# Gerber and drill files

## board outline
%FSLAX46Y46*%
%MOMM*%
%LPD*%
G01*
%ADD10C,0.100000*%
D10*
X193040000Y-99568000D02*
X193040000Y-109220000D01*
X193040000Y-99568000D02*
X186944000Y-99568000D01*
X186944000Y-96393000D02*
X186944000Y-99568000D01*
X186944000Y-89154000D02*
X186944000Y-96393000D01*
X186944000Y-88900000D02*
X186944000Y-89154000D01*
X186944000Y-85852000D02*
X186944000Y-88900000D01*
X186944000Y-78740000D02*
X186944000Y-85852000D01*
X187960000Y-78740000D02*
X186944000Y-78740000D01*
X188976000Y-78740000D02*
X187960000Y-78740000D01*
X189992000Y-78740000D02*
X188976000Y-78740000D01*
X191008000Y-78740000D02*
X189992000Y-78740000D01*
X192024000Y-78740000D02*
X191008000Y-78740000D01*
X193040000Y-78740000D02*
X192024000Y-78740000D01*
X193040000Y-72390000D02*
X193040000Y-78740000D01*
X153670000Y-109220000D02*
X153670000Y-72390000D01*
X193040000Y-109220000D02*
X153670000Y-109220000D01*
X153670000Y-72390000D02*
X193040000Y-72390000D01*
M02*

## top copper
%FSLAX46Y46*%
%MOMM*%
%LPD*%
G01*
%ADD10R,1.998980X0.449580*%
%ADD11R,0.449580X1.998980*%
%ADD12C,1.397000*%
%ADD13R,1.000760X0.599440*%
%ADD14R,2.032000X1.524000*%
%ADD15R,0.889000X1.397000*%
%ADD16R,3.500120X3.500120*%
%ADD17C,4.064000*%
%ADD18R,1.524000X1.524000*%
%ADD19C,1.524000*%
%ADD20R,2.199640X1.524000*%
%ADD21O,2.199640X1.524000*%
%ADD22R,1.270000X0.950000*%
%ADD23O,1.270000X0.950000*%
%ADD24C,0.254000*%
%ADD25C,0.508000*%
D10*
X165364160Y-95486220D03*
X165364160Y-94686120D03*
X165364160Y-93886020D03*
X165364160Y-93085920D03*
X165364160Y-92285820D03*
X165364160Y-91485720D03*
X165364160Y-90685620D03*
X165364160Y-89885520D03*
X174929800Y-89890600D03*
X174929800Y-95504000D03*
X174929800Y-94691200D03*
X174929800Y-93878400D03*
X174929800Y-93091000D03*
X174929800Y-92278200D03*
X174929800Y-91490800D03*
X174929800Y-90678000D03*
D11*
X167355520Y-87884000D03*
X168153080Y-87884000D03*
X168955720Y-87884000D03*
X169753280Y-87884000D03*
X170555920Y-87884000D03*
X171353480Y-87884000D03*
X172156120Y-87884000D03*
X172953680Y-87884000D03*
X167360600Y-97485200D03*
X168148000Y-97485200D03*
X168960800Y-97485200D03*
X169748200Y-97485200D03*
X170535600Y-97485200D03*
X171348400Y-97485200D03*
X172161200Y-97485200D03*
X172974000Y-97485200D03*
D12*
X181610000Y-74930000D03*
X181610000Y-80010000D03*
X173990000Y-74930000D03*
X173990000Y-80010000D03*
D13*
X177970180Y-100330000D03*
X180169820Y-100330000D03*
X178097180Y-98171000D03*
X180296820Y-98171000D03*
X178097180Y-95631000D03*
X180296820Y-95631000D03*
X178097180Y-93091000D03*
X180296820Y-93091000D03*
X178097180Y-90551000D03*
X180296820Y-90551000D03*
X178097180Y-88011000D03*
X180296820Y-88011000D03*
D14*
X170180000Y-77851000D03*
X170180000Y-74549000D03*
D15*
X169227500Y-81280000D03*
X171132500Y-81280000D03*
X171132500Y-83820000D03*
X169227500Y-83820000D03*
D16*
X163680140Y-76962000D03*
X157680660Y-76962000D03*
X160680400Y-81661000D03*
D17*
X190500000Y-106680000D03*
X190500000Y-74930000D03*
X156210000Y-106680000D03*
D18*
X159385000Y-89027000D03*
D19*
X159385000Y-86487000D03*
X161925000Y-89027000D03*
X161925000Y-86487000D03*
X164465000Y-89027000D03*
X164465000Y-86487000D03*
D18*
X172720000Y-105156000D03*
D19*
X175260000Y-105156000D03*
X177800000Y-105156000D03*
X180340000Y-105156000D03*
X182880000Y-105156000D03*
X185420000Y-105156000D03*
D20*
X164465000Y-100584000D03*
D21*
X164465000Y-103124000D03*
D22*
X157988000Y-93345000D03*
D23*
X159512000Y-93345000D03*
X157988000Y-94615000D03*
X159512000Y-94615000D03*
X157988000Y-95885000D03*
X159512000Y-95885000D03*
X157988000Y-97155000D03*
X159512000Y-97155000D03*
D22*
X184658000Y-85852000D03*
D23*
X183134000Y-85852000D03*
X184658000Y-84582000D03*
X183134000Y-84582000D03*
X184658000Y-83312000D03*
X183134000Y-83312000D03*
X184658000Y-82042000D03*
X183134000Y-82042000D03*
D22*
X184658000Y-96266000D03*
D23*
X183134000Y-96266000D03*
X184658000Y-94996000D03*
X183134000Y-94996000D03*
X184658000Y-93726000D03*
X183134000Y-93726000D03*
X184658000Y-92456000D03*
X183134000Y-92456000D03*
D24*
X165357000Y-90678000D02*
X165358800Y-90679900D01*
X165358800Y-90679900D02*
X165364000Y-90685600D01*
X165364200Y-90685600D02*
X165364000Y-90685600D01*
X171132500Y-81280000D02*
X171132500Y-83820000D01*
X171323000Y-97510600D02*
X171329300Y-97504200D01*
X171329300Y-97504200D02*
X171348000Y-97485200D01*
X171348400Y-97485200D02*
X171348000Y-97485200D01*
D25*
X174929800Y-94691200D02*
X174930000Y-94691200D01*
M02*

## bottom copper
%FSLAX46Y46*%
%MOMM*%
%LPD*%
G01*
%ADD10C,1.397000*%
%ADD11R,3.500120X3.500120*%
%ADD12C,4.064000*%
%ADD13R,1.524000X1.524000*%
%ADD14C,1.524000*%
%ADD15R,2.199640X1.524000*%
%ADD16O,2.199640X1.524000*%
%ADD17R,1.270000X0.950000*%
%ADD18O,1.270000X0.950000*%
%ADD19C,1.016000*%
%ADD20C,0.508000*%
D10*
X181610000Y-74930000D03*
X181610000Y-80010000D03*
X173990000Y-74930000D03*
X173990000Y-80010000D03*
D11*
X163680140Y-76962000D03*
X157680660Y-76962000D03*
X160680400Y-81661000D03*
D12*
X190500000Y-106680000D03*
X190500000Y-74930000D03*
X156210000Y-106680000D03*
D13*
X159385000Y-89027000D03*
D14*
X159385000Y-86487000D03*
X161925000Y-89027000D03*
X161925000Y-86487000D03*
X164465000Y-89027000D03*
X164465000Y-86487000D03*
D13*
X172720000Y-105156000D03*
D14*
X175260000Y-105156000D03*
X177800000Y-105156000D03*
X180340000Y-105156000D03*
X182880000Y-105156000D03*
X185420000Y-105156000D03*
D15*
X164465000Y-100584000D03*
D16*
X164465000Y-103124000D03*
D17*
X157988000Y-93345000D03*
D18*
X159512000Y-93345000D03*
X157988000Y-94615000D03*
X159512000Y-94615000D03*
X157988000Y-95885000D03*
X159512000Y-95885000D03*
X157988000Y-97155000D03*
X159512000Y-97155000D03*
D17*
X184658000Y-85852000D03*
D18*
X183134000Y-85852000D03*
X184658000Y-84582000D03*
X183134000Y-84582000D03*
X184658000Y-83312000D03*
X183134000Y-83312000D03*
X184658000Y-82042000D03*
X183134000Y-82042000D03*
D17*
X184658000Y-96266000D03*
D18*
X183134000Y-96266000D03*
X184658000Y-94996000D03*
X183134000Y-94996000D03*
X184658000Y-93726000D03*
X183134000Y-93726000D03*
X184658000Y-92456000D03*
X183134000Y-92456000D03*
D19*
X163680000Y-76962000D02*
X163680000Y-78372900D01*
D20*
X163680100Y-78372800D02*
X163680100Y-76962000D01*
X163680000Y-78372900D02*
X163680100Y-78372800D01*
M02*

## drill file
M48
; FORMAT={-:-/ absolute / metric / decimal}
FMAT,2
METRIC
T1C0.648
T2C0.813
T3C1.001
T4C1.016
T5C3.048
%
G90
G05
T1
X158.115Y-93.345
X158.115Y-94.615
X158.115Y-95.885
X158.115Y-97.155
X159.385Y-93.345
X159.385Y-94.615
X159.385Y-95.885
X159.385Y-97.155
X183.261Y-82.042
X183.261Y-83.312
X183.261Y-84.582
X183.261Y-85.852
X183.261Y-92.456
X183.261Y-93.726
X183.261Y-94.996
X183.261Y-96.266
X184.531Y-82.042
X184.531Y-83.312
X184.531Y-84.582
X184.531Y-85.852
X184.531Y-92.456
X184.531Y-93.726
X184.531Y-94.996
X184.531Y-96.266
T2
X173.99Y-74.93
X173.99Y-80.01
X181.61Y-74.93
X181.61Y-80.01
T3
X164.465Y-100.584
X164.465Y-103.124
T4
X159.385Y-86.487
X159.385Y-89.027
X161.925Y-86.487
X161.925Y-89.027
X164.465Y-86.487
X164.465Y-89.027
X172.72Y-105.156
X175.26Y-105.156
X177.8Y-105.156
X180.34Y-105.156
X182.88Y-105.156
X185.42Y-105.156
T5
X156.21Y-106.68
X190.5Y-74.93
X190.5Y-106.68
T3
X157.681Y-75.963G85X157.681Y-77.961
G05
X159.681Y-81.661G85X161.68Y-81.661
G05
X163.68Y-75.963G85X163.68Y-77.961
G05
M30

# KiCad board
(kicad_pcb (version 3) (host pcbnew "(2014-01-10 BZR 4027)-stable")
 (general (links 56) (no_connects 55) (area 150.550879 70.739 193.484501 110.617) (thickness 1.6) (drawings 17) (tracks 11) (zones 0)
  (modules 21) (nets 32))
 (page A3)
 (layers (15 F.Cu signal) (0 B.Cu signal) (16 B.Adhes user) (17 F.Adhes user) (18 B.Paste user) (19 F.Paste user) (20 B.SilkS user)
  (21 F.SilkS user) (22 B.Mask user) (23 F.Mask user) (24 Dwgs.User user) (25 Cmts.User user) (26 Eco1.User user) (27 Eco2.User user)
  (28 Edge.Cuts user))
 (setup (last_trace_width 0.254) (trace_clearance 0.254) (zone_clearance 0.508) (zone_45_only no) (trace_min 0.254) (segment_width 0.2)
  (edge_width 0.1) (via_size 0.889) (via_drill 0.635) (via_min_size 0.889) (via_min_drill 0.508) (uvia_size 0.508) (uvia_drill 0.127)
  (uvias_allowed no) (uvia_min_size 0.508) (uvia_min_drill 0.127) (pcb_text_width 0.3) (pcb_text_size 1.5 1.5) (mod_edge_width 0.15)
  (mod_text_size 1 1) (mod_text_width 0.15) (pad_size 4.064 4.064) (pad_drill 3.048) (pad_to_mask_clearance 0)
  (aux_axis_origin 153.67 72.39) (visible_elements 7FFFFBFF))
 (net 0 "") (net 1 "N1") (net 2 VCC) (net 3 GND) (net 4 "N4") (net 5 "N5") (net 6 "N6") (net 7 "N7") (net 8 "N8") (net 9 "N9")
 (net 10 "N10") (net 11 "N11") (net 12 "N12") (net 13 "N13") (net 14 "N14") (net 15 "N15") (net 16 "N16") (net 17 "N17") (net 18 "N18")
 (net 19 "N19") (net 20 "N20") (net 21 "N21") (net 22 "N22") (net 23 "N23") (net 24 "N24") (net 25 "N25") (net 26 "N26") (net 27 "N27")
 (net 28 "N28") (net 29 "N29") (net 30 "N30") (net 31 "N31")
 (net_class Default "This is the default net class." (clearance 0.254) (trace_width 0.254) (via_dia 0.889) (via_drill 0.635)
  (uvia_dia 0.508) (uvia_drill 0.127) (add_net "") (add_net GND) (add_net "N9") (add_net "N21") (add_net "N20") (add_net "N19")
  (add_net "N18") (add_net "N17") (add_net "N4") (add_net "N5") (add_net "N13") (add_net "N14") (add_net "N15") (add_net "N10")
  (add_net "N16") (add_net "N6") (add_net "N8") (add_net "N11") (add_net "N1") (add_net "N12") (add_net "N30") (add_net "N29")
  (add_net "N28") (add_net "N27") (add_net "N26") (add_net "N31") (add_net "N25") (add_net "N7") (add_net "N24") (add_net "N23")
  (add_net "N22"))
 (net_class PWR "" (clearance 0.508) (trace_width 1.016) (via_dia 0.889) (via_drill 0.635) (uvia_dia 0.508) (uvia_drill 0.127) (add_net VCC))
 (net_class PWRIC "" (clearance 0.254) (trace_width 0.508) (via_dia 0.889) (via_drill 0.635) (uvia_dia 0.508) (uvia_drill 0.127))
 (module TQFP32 (layer F.Cu) (at 170.18 92.71)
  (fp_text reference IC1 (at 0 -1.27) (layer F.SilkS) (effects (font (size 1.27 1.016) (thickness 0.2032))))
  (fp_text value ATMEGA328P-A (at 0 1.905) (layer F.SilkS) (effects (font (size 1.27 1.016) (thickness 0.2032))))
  (pad 8 smd rect (at -4.81584 2.77622) (size 1.99898 0.44958) (layers F.Cu F.Paste F.Mask) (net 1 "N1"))
  (pad 7 smd rect (at -4.81584 1.97612) (size 1.99898 0.44958) (layers F.Cu F.Paste F.Mask))
  (pad 6 smd rect (at -4.81584 1.17602) (size 1.99898 0.44958) (layers F.Cu F.Paste F.Mask) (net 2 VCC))
  (pad 5 smd rect (at -4.81584 0.37592) (size 1.99898 0.44958) (layers F.Cu F.Paste F.Mask) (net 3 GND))
  (pad 4 smd rect (at -4.81584 -0.42418) (size 1.99898 0.44958) (layers F.Cu F.Paste F.Mask) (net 2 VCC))
  (pad 3 smd rect (at -4.81584 -1.22428) (size 1.99898 0.44958) (layers F.Cu F.Paste F.Mask) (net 3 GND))
  (pad 2 smd rect (at -4.81584 -2.02438) (size 1.99898 0.44958) (layers F.Cu F.Paste F.Mask) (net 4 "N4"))
  (pad 1 smd rect (at -4.81584 -2.82448) (size 1.99898 0.44958) (layers F.Cu F.Paste F.Mask) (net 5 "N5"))
  (pad 24 smd rect (at 4.7498 -2.8194) (size 1.99898 0.44958) (layers F.Cu F.Paste F.Mask) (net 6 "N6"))
  (pad 17 smd rect (at 4.7498 2.794) (size 1.99898 0.44958) (layers F.Cu F.Paste F.Mask) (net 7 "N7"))
  (pad 18 smd rect (at 4.7498 1.9812) (size 1.99898 0.44958) (layers F.Cu F.Paste F.Mask) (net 2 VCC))
  (pad 19 smd rect (at 4.7498 1.1684) (size 1.99898 0.44958) (layers F.Cu F.Paste F.Mask))
  (pad 20 smd rect (at 4.7498 0.381) (size 1.99898 0.44958) (layers F.Cu F.Paste F.Mask))
  (pad 21 smd rect (at 4.7498 -0.4318) (size 1.99898 0.44958) (layers F.Cu F.Paste F.Mask) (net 3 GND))
  (pad 22 smd rect (at 4.7498 -1.2192) (size 1.99898 0.44958) (layers F.Cu F.Paste F.Mask))
  (pad 23 smd rect (at 4.7498 -2.032) (size 1.99898 0.44958) (layers F.Cu F.Paste F.Mask) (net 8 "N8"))
  (pad 32 smd rect (at -2.82448 -4.826) (size 0.44958 1.99898) (layers F.Cu F.Paste F.Mask) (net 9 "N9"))
  (pad 31 smd rect (at -2.02692 -4.826) (size 0.44958 1.99898) (layers F.Cu F.Paste F.Mask) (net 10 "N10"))
  (pad 30 smd rect (at -1.22428 -4.826) (size 0.44958 1.99898) (layers F.Cu F.Paste F.Mask) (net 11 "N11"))
  (pad 29 smd rect (at -0.42672 -4.826) (size 0.44958 1.99898) (layers F.Cu F.Paste F.Mask) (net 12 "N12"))
  (pad 28 smd rect (at 0.37592 -4.826) (size 0.44958 1.99898) (layers F.Cu F.Paste F.Mask) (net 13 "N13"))
  (pad 27 smd rect (at 1.17348 -4.826) (size 0.44958 1.99898) (layers F.Cu F.Paste F.Mask) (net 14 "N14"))
  (pad 26 smd rect (at 1.97612 -4.826) (size 0.44958 1.99898) (layers F.Cu F.Paste F.Mask) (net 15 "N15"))
  (pad 25 smd rect (at 2.77368 -4.826) (size 0.44958 1.99898) (layers F.Cu F.Paste F.Mask) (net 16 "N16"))
  (pad 9 smd rect (at -2.8194 4.7752) (size 0.44958 1.99898) (layers F.Cu F.Paste F.Mask) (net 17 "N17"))
  (pad 10 smd rect (at -2.032 4.7752) (size 0.44958 1.99898) (layers F.Cu F.Paste F.Mask) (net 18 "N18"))
  (pad 11 smd rect (at -1.2192 4.7752) (size 0.44958 1.99898) (layers F.Cu F.Paste F.Mask) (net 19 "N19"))
  (pad 12 smd rect (at -0.4318 4.7752) (size 0.44958 1.99898) (layers F.Cu F.Paste F.Mask) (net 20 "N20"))
  (pad 13 smd rect (at 0.3556 4.7752) (size 0.44958 1.99898) (layers F.Cu F.Paste F.Mask) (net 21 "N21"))
  (pad 14 smd rect (at 1.1684 4.7752) (size 0.44958 1.99898) (layers F.Cu F.Paste F.Mask) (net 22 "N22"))
  (pad 15 smd rect (at 1.9812 4.7752) (size 0.44958 1.99898) (layers F.Cu F.Paste F.Mask) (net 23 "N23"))
  (pad 16 smd rect (at 2.794 4.7752) (size 0.44958 1.99898) (layers F.Cu F.Paste F.Mask) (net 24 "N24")))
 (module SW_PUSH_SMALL (layer F.Cu) (at 177.8 77.47)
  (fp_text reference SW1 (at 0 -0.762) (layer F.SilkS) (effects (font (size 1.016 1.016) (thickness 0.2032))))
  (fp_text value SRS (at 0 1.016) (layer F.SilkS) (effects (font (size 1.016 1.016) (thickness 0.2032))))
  (pad 1 thru_hole circle (at 3.81 -2.54) (size 1.397 1.397) (drill 0.8128) (layers *.Cu *.Mask F.SilkS) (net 1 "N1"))
  (pad 2 thru_hole circle (at 3.81 2.54) (size 1.397 1.397) (drill 0.8128) (layers *.Cu *.Mask F.SilkS) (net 3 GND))
  (pad 1 thru_hole circle (at -3.81 -2.54) (size 1.397 1.397) (drill 0.8128) (layers *.Cu *.Mask F.SilkS) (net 1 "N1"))
  (pad 2 thru_hole circle (at -3.81 2.54) (size 1.397 1.397) (drill 0.8128) (layers *.Cu *.Mask F.SilkS) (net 3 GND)))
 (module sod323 (layer F.Cu) (at 179.07 100.33 180)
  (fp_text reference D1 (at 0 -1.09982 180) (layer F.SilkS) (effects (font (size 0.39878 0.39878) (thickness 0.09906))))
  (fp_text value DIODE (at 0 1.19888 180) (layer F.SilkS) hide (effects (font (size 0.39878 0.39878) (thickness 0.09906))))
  (pad 2 smd rect (at 1.09982 0 180) (size 1.00076 0.59944) (layers F.Cu F.Paste F.Mask) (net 20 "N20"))
  (pad 1 smd rect (at -1.09982 0 180) (size 1.00076 0.59944) (layers F.Cu F.Paste F.Mask) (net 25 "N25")))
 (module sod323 (layer F.Cu) (at 179.197 98.171 180)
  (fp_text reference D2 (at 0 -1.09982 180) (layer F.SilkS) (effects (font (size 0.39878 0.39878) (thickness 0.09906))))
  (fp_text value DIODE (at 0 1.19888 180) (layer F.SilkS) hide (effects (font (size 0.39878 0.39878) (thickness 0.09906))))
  (pad 2 smd rect (at 1.09982 0 180) (size 1.00076 0.59944) (layers F.Cu F.Paste F.Mask) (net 21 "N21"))
  (pad 1 smd rect (at -1.09982 0 180) (size 1.00076 0.59944) (layers F.Cu F.Paste F.Mask) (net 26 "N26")))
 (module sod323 (layer F.Cu) (at 179.197 95.631 180)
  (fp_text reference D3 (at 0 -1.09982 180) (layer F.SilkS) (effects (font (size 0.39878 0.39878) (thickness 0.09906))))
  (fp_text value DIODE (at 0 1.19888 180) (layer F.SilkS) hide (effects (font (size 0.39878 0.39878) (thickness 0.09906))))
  (pad 2 smd rect (at 1.09982 0 180) (size 1.00076 0.59944) (layers F.Cu F.Paste F.Mask) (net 22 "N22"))
  (pad 1 smd rect (at -1.09982 0 180) (size 1.00076 0.59944) (layers F.Cu F.Paste F.Mask) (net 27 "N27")))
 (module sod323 (layer F.Cu) (at 179.197 93.091 180)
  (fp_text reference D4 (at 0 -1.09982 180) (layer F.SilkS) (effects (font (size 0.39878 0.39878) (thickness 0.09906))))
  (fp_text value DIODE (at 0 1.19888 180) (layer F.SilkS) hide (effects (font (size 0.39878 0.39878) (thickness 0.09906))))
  (pad 2 smd rect (at 1.09982 0 180) (size 1.00076 0.59944) (layers F.Cu F.Paste F.Mask) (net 23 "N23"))
  (pad 1 smd rect (at -1.09982 0 180) (size 1.00076 0.59944) (layers F.Cu F.Paste F.Mask) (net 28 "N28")))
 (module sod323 (layer F.Cu) (at 179.197 90.551 180)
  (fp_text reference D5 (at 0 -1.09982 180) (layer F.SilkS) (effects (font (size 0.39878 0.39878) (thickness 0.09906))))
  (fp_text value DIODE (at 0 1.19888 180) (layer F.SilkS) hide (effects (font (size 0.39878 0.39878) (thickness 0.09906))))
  (pad 2 smd rect (at 1.09982 0 180) (size 1.00076 0.59944) (layers F.Cu F.Paste F.Mask) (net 24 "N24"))
  (pad 1 smd rect (at -1.09982 0 180) (size 1.00076 0.59944) (layers F.Cu F.Paste F.Mask) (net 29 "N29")))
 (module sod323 (layer F.Cu) (at 179.197 88.011 180)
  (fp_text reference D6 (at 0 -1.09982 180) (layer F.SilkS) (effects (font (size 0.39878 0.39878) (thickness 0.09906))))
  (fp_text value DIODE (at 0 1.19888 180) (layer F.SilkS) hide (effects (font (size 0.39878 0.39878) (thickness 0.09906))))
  (pad 2 smd rect (at 1.09982 0 180) (size 1.00076 0.59944) (layers F.Cu F.Paste F.Mask) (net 7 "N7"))
  (pad 1 smd rect (at -1.09982 0 180) (size 1.00076 0.59944) (layers F.Cu F.Paste F.Mask) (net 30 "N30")))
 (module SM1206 (layer F.Cu) (at 170.18 76.2 90)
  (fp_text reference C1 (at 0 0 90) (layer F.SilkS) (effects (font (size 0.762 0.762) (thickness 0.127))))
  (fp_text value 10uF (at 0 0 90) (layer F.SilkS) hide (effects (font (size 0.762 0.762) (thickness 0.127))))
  (pad 1 smd rect (at -1.651 0 90) (size 1.524 2.032) (layers F.Cu F.Paste F.Mask) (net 2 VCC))
  (pad 2 smd rect (at 1.651 0 90) (size 1.524 2.032) (layers F.Cu F.Paste F.Mask) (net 3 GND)))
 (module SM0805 (layer F.Cu) (at 170.18 81.28)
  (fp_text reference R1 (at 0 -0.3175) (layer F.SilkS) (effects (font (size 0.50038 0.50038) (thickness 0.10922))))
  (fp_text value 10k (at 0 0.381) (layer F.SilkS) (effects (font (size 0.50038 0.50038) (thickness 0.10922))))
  (pad 1 smd rect (at -0.9525 0) (size 0.889 1.397) (layers F.Cu F.Paste F.Mask) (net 2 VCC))
  (pad 2 smd rect (at 0.9525 0) (size 0.889 1.397) (layers F.Cu F.Paste F.Mask) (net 12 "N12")))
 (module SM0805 (layer F.Cu) (at 170.18 83.82 180)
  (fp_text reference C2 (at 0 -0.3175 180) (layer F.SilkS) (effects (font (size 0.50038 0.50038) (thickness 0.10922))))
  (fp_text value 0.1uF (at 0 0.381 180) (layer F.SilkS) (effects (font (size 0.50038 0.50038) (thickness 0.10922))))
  (pad 1 smd rect (at -0.9525 0 180) (size 0.889 1.397) (layers F.Cu F.Paste F.Mask) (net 12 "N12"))
  (pad 2 smd rect (at 0.9525 0 180) (size 0.889 1.397) (layers F.Cu F.Paste F.Mask) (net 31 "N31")))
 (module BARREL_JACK (layer F.Cu) (at 157.48 76.962)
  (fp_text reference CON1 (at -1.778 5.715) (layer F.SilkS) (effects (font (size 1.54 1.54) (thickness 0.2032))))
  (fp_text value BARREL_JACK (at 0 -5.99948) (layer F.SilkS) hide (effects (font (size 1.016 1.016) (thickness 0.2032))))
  (pad 1 thru_hole rect (at 6.20014 0) (size 3.50012 3.50012) (drill oval 1.00076 2.99974) (layers *.Cu *.Mask F.SilkS) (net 2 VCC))
  (pad 2 thru_hole rect (at 0.20066 0) (size 3.50012 3.50012) (drill oval 1.00076 2.99974) (layers *.Cu *.Mask F.SilkS) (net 3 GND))
  (pad 3 thru_hole rect (at 3.2004 4.699) (size 3.50012 3.50012) (drill oval 2.99974 1.00076) (layers *.Cu *.Mask F.SilkS) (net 3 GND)))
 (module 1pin (layer F.Cu) (at 190.5 106.68)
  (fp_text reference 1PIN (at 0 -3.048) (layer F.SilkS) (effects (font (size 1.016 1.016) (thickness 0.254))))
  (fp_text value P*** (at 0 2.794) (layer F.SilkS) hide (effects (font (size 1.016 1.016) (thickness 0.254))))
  (pad 1 thru_hole circle (at 0 0) (size 4.064 4.064) (drill 3.048) (layers *.Cu *.Mask F.SilkS)))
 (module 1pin (layer F.Cu) (at 190.5 74.93)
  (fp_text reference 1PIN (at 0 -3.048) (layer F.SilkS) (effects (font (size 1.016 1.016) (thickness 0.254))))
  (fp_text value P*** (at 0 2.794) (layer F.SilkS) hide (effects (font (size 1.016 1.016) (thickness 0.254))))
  (pad 1 thru_hole circle (at 0 0) (size 4.064 4.064) (drill 3.048) (layers *.Cu *.Mask F.SilkS)))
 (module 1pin (layer F.Cu) (at 156.21 106.68)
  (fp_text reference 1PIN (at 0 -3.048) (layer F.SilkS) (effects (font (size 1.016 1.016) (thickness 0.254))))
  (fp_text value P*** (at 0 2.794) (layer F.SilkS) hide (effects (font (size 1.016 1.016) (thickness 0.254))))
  (pad 1 thru_hole circle (at 0 0) (size 4.064 4.064) (drill 3.048) (layers *.Cu *.Mask F.SilkS) (clearance 1)))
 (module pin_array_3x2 (layer F.Cu) (at 161.925 87.757)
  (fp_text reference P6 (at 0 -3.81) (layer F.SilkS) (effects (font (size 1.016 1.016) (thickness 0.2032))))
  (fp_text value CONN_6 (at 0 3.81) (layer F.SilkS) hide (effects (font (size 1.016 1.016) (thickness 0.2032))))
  (pad 1 thru_hole rect (at -2.54 1.27) (size 1.524 1.524) (drill 1.016) (layers *.Cu *.Mask F.SilkS) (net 24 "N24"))
  (pad 2 thru_hole circle (at -2.54 -1.27) (size 1.524 1.524) (drill 1.016) (layers *.Cu *.Mask F.SilkS) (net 2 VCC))
  (pad 3 thru_hole circle (at 0 1.27) (size 1.524 1.524) (drill 1.016) (layers *.Cu *.Mask F.SilkS) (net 7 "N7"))
  (pad 4 thru_hole circle (at 0 -1.27) (size 1.524 1.524) (drill 1.016) (layers *.Cu *.Mask F.SilkS) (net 23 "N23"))
  (pad 5 thru_hole circle (at 2.54 1.27) (size 1.524 1.524) (drill 1.016) (layers *.Cu *.Mask F.SilkS) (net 12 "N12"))
  (pad 6 thru_hole circle (at 2.54 -1.27) (size 1.524 1.524) (drill 1.016) (layers *.Cu *.Mask F.SilkS) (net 3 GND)))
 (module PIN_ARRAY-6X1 (layer F.Cu) (at 179.07 105.156)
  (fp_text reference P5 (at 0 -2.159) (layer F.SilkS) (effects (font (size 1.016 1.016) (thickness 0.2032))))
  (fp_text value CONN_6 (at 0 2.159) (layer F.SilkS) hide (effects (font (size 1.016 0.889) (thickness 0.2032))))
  (pad 1 thru_hole rect (at -6.35 0) (size 1.524 1.524) (drill 1.016) (layers *.Cu *.Mask F.SilkS) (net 31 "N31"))
  (pad 2 thru_hole circle (at -3.81 0) (size 1.524 1.524) (drill 1.016) (layers *.Cu *.Mask F.SilkS) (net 10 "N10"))
  (pad 3 thru_hole circle (at -1.27 0) (size 1.524 1.524) (drill 1.016) (layers *.Cu *.Mask F.SilkS) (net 11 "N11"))
  (pad 4 thru_hole circle (at 1.27 0) (size 1.524 1.524) (drill 1.016) (layers *.Cu *.Mask F.SilkS) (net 2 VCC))
  (pad 5 thru_hole circle (at 3.81 0) (size 1.524 1.524) (drill 1.016) (layers *.Cu *.Mask F.SilkS) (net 3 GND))
  (pad 6 thru_hole circle (at 6.35 0) (size 1.524 1.524) (drill 1.016) (layers *.Cu *.Mask F.SilkS) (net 3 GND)))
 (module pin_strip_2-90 (layer F.Cu) (at 164.465 101.854 270)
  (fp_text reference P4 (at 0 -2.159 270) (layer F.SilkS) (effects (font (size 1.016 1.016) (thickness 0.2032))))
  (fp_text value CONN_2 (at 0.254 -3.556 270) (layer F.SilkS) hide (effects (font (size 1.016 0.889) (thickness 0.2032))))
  (pad 1 thru_hole rect (at -1.27 0 270) (size 1.524 2.19964) (drill 1.00076) (layers *.Cu *.Mask F.SilkS) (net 2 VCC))
  (pad 2 thru_hole oval (at 1.27 0 270) (size 1.524 2.19964) (drill 1.00076) (layers *.Cu *.Mask F.SilkS) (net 3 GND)))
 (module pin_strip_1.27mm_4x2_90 (layer F.Cu) (at 158.75 95.25 270)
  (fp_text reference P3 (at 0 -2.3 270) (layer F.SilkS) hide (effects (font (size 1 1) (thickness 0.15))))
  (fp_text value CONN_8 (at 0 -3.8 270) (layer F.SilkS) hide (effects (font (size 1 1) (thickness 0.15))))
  (pad 1 thru_hole rect (at -1.905 0.635 270) (size 0.95 1.27) (drill 0.6477 (offset 0 0.127)) (layers *.Cu *.Mask F.SilkS) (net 11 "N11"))
  (pad 2 thru_hole oval (at -1.905 -0.635 270) (size 0.95 1.27) (drill 0.6477 (offset 0 -0.127)) (layers *.Cu *.Mask F.SilkS) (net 10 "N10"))
  (pad 3 thru_hole oval (at -0.635 0.635 270) (size 0.95 1.27) (drill 0.6477 (offset 0 0.127)) (layers *.Cu *.Mask F.SilkS) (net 9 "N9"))
  (pad 4 thru_hole oval (at -0.635 -0.635 270) (size 0.95 1.27) (drill 0.6477 (offset 0 -0.127)) (layers *.Cu *.Mask F.SilkS) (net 5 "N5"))
  (pad 5 thru_hole oval (at 0.635 0.635 270) (size 0.95 1.27) (drill 0.6477 (offset 0 0.127)) (layers *.Cu *.Mask F.SilkS) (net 4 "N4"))
  (pad 6 thru_hole oval (at 0.635 -0.635 270) (size 0.95 1.27) (drill 0.6477 (offset 0 -0.127)) (layers *.Cu *.Mask F.SilkS) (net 17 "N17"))
  (pad 7 thru_hole oval (at 1.905 0.635 270) (size 0.95 1.27) (drill 0.6477 (offset 0 0.127)) (layers *.Cu *.Mask F.SilkS) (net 18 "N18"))
  (pad 8 thru_hole oval (at 1.905 -0.635 270) (size 0.95 1.27) (drill 0.6477 (offset 0 -0.127)) (layers *.Cu *.Mask F.SilkS) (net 19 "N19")))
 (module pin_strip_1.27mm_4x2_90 (layer F.Cu) (at 183.896 83.947 90)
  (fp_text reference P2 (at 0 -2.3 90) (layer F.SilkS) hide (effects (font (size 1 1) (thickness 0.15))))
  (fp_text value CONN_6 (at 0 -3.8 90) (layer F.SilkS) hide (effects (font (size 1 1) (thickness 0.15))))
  (pad 1 thru_hole rect (at -1.905 0.635 90) (size 0.95 1.27) (drill 0.6477 (offset 0 0.127)) (layers *.Cu *.Mask F.SilkS) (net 8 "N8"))
  (pad 2 thru_hole oval (at -1.905 -0.635 90) (size 0.95 1.27) (drill 0.6477 (offset 0 -0.127)) (layers *.Cu *.Mask F.SilkS) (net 6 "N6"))
  (pad 3 thru_hole oval (at -0.635 0.635 90) (size 0.95 1.27) (drill 0.6477 (offset 0 0.127)) (layers *.Cu *.Mask F.SilkS) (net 16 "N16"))
  (pad 4 thru_hole oval (at -0.635 -0.635 90) (size 0.95 1.27) (drill 0.6477 (offset 0 -0.127)) (layers *.Cu *.Mask F.SilkS) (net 15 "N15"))
  (pad 5 thru_hole oval (at 0.635 0.635 90) (size 0.95 1.27) (drill 0.6477 (offset 0 0.127)) (layers *.Cu *.Mask F.SilkS) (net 14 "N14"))
  (pad 6 thru_hole oval (at 0.635 -0.635 90) (size 0.95 1.27) (drill 0.6477 (offset 0 -0.127)) (layers *.Cu *.Mask F.SilkS) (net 13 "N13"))
  (pad 7 thru_hole oval (at 1.905 0.635 90) (size 0.95 1.27) (drill 0.6477 (offset 0 0.127)) (layers *.Cu *.Mask F.SilkS))
  (pad 8 thru_hole oval (at 1.905 -0.635 90) (size 0.95 1.27) (drill 0.6477 (offset 0 -0.127)) (layers *.Cu *.Mask F.SilkS)))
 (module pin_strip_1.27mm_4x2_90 (layer F.Cu) (at 183.896 94.361 90)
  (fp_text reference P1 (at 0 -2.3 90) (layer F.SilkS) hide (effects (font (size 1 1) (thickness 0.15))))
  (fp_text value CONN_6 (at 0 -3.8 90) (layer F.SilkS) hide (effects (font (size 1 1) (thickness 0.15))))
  (pad 1 thru_hole rect (at -1.905 0.635 90) (size 0.95 1.27) (drill 0.6477 (offset 0 0.127)) (layers *.Cu *.Mask F.SilkS) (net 25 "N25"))
  (pad 2 thru_hole oval (at -1.905 -0.635 90) (size 0.95 1.27) (drill 0.6477 (offset 0 -0.127)) (layers *.Cu *.Mask F.SilkS) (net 26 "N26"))
  (pad 3 thru_hole oval (at -0.635 0.635 90) (size 0.95 1.27) (drill 0.6477 (offset 0 0.127)) (layers *.Cu *.Mask F.SilkS) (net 27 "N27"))
  (pad 4 thru_hole oval (at -0.635 -0.635 90) (size 0.95 1.27) (drill 0.6477 (offset 0 -0.127)) (layers *.Cu *.Mask F.SilkS) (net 28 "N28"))
  (pad 5 thru_hole oval (at 0.635 0.635 90) (size 0.95 1.27) (drill 0.6477 (offset 0 0.127)) (layers *.Cu *.Mask F.SilkS) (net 29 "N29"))
  (pad 6 thru_hole oval (at 0.635 -0.635 90) (size 0.95 1.27) (drill 0.6477 (offset 0 -0.127)) (layers *.Cu *.Mask F.SilkS) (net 30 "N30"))
  (pad 7 thru_hole oval (at 1.905 0.635 90) (size 0.95 1.27) (drill 0.6477 (offset 0 0.127)) (layers *.Cu *.Mask F.SilkS))
  (pad 8 thru_hole oval (at 1.905 -0.635 90) (size 0.95 1.27) (drill 0.6477 (offset 0 -0.127)) (layers *.Cu *.Mask F.SilkS)))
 (gr_line (start 193.04 99.568) (end 193.04 109.22) (angle 90) (layer Edge.Cuts) (width 0.1))
 (gr_line (start 193.04 99.568) (end 186.944 99.568) (angle 90) (layer Edge.Cuts) (width 0.1))
 (gr_line (start 186.944 96.393) (end 186.944 99.568) (angle 90) (layer Edge.Cuts) (width 0.1))
 (gr_line (start 186.944 89.154) (end 186.944 96.393) (angle 90) (layer Edge.Cuts) (width 0.1))
 (gr_line (start 186.944 88.9) (end 186.944 89.154) (angle 90) (layer Edge.Cuts) (width 0.1))
 (gr_line (start 186.944 85.852) (end 186.944 88.9) (angle 90) (layer Edge.Cuts) (width 0.1))
 (gr_line (start 186.944 78.74) (end 186.944 85.852) (angle 90) (layer Edge.Cuts) (width 0.1))
 (gr_line (start 187.96 78.74) (end 186.944 78.74) (angle 90) (layer Edge.Cuts) (width 0.1))
 (gr_line (start 188.976 78.74) (end 187.96 78.74) (angle 90) (layer Edge.Cuts) (width 0.1))
 (gr_line (start 189.992 78.74) (end 188.976 78.74) (angle 90) (layer Edge.Cuts) (width 0.1))
 (gr_line (start 191.008 78.74) (end 189.992 78.74) (angle 90) (layer Edge.Cuts) (width 0.1))
 (gr_line (start 192.024 78.74) (end 191.008 78.74) (angle 90) (layer Edge.Cuts) (width 0.1))
 (gr_line (start 193.04 78.74) (end 192.024 78.74) (angle 90) (layer Edge.Cuts) (width 0.1))
 (gr_line (start 193.04 72.39) (end 193.04 78.74) (angle 90) (layer Edge.Cuts) (width 0.1))
 (gr_line (start 153.67 109.22) (end 153.67 72.39) (angle 90) (layer Edge.Cuts) (width 0.1))
 (gr_line (start 193.04 109.22) (end 153.67 109.22) (angle 90) (layer Edge.Cuts) (width 0.1))
 (gr_line (start 153.67 72.39) (end 193.04 72.39) (angle 90) (layer Edge.Cuts) (width 0.1))
 (segment (start 165.357 90.678) (end 165.3588 90.6799) (width 0.254) (layer F.Cu) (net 4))
 (segment (start 165.3588 90.6799) (end 165.364 90.6856) (width 0.254) (layer F.Cu) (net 4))
 (segment (start 165.3642 90.6856) (end 165.364 90.6856) (width 0.254) (layer F.Cu) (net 4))
 (segment (start 171.1325 81.28) (end 171.1325 83.82) (width 0.254) (layer F.Cu) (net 12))
 (segment (start 171.323 97.5106) (end 171.3293 97.5042) (width 0.254) (layer F.Cu) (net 22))
 (segment (start 171.3293 97.5042) (end 171.348 97.4852) (width 0.254) (layer F.Cu) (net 22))
 (segment (start 171.3484 97.4852) (end 171.348 97.4852) (width 0.254) (layer F.Cu) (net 22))
 (segment (start 174.9298 94.6912) (end 174.93 94.6912) (width 0.508) (layer F.Cu) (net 2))
 (segment (start 163.68 76.962) (end 163.68 78.3729) (width 1.016) (layer B.Cu) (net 2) (status 30))
 (segment (start 163.6801 78.3728) (end 163.6801 76.962) (width 0.508) (layer B.Cu) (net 2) (status 30))
 (segment (start 163.68 78.3729) (end 163.6801 78.3728) (width 0.508) (layer B.Cu) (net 2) (status 30)))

